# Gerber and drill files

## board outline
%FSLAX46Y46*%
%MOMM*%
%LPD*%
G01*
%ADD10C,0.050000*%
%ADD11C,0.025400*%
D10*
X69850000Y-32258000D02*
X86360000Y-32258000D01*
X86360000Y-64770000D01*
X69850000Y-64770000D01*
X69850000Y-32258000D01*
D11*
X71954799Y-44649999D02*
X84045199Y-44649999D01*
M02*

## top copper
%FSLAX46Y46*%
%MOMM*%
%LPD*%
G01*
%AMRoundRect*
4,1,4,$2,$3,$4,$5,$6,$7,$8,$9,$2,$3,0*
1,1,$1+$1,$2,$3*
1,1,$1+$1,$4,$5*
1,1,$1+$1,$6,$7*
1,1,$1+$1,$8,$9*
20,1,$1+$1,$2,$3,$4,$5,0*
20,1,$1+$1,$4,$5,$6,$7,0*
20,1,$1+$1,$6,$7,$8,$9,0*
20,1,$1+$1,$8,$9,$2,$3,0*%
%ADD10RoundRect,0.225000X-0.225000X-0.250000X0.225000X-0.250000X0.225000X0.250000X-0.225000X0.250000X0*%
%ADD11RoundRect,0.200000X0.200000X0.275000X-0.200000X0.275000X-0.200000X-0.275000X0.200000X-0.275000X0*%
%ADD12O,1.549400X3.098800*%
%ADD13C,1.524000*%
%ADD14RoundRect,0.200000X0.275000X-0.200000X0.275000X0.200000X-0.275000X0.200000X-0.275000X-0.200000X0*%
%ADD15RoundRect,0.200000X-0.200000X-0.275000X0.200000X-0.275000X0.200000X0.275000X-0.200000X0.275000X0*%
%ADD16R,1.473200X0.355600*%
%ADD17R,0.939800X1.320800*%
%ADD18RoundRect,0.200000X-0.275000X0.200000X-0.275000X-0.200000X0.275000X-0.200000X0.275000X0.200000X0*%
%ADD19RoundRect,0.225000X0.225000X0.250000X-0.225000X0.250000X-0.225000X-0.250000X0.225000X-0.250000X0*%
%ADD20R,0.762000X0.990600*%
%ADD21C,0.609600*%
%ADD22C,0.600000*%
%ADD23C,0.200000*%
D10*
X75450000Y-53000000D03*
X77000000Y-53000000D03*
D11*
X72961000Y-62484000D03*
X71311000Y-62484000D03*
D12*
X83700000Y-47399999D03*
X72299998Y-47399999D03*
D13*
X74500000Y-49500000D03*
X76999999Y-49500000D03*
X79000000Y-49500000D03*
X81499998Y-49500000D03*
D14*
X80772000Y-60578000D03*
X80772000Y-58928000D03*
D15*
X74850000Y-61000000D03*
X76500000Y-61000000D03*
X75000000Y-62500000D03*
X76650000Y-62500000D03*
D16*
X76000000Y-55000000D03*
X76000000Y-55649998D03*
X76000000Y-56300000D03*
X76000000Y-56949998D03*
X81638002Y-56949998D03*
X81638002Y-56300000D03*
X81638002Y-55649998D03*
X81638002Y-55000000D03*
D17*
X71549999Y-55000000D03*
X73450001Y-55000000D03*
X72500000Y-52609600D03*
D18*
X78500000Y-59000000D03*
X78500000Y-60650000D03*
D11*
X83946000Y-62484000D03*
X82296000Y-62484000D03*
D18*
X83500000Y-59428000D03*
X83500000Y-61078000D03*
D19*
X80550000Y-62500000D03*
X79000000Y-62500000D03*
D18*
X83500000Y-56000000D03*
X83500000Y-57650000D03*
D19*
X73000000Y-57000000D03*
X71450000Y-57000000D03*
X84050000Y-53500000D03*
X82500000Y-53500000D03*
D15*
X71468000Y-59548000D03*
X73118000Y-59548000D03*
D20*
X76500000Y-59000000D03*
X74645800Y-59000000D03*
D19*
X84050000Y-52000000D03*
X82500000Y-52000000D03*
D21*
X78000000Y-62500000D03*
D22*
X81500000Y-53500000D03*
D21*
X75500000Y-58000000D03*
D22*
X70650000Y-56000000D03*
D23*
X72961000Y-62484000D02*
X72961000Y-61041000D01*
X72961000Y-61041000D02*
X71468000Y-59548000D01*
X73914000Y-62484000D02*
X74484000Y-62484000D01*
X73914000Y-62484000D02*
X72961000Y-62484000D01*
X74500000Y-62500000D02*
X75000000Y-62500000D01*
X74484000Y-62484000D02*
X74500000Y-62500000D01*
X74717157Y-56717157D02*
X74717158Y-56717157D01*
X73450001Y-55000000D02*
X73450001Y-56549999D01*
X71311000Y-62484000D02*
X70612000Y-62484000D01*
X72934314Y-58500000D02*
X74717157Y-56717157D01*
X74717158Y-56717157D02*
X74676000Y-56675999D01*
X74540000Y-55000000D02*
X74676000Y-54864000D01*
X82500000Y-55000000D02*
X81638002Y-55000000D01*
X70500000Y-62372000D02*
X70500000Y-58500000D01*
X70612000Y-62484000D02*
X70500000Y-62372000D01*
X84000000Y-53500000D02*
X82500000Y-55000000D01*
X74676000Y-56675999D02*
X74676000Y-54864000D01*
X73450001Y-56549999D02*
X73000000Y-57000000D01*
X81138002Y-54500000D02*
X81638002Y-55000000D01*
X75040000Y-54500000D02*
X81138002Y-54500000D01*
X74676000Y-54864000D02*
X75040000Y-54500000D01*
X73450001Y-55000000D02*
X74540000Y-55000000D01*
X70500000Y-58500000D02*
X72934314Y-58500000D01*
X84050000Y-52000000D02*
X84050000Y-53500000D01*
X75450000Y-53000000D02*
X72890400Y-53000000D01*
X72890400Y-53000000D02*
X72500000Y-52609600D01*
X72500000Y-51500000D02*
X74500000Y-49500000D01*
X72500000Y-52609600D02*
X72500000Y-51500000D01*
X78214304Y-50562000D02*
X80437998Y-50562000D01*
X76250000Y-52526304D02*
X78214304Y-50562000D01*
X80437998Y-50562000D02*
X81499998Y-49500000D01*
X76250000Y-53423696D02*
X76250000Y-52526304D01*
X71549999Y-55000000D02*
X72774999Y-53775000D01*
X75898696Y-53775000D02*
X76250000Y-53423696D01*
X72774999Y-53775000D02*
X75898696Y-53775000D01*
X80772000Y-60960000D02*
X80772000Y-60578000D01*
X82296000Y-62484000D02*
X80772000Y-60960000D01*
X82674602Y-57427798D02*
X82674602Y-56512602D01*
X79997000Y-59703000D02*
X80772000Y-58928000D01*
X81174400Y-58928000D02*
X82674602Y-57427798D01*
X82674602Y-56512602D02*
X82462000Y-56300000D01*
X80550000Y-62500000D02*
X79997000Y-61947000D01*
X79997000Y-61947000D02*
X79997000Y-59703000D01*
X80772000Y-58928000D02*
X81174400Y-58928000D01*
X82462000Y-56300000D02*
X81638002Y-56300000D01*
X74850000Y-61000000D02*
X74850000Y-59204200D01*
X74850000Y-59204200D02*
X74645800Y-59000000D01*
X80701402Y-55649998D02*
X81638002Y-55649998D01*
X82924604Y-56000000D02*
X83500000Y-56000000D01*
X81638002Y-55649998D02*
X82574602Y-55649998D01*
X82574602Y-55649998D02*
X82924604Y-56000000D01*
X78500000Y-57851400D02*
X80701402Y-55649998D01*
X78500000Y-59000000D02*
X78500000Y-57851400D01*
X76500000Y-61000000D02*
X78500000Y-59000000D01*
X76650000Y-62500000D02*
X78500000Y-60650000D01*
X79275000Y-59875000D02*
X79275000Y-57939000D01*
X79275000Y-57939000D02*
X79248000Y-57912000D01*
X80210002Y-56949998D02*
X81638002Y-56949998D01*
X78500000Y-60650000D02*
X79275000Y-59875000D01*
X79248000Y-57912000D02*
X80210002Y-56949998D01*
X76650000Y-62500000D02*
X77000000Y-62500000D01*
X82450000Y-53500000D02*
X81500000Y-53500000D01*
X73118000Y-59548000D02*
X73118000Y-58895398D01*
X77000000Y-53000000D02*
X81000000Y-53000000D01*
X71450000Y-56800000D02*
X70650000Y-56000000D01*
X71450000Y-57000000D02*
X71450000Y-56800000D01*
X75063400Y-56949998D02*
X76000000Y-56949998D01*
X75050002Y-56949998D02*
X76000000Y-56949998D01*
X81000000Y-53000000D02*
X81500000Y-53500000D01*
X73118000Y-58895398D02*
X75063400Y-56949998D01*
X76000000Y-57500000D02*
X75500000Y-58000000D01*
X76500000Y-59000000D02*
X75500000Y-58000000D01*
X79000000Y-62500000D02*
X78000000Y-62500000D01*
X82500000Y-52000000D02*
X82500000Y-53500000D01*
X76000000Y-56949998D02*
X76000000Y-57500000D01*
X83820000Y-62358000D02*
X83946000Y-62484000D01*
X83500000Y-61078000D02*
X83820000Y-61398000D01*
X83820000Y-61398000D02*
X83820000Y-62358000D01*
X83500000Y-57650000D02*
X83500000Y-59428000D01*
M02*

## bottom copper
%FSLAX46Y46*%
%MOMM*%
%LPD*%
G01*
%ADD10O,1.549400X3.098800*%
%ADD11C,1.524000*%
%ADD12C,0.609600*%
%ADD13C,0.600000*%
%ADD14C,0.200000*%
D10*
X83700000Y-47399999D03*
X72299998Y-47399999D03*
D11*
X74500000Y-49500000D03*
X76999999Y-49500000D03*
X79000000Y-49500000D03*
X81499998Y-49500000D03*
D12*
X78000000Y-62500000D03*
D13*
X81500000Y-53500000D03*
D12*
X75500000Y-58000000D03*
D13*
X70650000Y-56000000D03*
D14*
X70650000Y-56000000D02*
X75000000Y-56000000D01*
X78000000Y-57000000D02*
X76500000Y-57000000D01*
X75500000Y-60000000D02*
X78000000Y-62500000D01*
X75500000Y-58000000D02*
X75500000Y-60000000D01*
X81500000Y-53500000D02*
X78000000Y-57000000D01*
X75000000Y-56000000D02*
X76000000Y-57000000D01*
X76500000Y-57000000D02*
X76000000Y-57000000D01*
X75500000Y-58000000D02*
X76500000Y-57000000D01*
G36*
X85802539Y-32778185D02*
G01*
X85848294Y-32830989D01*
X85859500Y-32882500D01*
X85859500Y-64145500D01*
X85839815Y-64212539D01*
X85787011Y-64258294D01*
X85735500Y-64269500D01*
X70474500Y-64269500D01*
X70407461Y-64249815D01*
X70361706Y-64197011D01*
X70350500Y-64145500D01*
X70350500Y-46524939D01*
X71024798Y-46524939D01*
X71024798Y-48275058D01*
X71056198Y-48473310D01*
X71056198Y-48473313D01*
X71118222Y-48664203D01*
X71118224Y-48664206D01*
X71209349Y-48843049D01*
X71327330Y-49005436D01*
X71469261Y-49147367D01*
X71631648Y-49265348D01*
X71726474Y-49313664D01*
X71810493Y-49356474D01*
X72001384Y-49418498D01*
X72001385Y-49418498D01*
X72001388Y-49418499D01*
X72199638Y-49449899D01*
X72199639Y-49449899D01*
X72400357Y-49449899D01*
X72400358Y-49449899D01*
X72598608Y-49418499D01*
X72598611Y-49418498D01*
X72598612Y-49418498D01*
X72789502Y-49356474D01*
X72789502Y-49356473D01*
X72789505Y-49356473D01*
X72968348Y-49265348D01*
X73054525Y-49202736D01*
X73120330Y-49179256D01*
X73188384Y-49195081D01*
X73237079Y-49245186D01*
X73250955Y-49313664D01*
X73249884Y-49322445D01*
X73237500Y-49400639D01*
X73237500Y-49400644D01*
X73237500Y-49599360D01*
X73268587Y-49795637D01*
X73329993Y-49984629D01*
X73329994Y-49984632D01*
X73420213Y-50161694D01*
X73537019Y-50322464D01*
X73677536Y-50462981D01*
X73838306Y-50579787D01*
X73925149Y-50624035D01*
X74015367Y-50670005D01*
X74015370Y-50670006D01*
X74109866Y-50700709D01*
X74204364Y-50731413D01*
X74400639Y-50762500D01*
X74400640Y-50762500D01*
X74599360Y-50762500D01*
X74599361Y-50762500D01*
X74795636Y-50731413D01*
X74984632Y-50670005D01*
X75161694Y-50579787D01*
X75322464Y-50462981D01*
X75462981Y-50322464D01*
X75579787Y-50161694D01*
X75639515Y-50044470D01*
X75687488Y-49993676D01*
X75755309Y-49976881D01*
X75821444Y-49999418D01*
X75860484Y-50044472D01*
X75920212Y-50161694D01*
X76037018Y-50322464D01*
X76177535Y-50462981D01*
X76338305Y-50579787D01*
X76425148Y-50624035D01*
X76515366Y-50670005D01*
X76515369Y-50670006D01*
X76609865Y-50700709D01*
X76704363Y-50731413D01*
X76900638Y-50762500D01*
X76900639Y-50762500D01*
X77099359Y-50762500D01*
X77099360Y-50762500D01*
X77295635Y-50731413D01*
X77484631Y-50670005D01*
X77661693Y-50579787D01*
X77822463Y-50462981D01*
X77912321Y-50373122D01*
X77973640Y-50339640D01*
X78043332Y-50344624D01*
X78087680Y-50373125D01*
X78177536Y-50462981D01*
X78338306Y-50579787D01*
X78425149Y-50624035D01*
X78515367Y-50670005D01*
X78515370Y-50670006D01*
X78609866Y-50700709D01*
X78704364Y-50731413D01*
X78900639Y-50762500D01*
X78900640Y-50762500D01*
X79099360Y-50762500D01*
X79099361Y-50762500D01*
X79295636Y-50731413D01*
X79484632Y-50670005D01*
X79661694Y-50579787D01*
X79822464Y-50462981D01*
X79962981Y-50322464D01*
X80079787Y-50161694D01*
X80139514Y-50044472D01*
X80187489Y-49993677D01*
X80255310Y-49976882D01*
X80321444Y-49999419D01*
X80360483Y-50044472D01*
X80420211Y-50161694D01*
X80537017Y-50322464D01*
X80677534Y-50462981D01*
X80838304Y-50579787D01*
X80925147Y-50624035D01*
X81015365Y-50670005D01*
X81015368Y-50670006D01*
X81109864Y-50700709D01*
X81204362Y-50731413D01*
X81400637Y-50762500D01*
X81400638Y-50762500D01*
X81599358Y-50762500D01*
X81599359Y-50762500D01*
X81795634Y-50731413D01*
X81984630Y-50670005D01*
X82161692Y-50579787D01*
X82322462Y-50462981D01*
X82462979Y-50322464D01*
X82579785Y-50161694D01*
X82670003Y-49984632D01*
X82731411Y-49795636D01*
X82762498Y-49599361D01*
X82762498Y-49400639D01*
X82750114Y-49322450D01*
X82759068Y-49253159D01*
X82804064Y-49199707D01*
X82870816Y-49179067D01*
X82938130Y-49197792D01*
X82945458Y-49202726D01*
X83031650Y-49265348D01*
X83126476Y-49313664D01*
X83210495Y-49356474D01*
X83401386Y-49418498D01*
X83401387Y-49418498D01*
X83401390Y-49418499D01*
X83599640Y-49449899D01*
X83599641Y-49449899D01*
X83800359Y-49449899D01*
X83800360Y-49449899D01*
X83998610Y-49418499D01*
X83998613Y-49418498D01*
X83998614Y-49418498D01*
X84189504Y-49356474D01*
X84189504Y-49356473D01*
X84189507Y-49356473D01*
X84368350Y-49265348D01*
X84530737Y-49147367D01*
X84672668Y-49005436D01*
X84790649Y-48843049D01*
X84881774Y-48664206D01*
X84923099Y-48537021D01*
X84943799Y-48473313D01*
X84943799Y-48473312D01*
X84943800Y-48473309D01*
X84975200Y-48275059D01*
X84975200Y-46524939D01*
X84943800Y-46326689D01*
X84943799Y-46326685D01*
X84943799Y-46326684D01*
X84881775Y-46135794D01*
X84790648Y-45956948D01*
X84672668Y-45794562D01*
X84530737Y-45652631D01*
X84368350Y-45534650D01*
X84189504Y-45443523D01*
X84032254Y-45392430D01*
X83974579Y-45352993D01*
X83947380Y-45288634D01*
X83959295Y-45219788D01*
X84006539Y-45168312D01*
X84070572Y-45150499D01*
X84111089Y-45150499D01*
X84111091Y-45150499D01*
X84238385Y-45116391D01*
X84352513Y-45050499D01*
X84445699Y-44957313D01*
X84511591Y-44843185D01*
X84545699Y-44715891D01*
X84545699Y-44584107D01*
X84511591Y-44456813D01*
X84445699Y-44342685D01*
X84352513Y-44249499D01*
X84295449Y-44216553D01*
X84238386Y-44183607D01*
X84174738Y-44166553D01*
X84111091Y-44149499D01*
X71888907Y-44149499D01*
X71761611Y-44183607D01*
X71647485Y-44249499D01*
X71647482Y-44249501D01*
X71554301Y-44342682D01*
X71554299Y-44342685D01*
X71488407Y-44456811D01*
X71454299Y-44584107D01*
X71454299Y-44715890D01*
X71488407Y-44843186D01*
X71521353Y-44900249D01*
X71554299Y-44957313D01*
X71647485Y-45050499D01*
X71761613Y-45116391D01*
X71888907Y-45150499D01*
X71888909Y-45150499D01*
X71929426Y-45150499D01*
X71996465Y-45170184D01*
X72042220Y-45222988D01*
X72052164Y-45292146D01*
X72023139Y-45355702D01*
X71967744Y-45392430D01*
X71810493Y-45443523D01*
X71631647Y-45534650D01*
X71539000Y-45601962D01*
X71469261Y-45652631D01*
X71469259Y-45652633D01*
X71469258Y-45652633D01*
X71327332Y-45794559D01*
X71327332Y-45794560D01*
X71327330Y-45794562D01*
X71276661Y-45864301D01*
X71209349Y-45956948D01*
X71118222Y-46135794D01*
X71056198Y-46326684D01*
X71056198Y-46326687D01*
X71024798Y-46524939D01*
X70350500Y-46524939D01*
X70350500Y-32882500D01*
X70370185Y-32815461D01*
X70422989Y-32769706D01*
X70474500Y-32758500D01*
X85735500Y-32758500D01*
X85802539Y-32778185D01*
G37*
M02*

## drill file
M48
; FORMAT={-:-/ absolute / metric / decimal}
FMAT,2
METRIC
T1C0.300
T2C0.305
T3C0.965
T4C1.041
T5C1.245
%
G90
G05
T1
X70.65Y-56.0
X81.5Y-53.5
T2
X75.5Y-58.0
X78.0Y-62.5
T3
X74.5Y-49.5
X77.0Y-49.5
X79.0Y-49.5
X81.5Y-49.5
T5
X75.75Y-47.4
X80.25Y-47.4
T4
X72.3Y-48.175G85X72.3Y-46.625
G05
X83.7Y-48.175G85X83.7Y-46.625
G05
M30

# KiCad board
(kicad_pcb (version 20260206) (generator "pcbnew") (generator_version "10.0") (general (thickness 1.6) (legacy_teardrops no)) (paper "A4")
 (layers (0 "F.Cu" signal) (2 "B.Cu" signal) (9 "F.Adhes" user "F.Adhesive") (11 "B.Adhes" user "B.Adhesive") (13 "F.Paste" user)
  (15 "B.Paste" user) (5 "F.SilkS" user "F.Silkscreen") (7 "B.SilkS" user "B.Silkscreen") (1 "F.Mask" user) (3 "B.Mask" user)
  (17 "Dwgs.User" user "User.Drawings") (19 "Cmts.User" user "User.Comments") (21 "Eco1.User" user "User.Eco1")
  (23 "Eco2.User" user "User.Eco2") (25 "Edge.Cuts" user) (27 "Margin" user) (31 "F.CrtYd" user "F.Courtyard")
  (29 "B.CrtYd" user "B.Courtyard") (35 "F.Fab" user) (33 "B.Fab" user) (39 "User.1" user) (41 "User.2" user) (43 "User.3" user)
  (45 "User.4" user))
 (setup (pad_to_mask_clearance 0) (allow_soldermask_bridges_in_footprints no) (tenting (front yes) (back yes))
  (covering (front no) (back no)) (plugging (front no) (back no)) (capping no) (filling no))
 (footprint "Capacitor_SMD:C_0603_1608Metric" (layer "F.Cu") (at 76.225 53)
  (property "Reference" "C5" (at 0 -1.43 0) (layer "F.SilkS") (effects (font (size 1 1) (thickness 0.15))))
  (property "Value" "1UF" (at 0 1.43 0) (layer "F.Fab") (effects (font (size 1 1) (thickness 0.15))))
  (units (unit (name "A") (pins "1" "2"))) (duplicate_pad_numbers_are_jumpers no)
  (pad "1" smd roundrect (at -0.775 0) (size 0.9 0.95) (layers "F.Cu" "F.Mask" "F.Paste") (roundrect_rratio 0.25) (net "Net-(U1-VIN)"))
  (pad "2" smd roundrect (at 0.775 0) (size 0.9 0.95) (layers "F.Cu" "F.Mask" "F.Paste") (roundrect_rratio 0.25) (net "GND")))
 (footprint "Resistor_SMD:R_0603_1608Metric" (layer "F.Cu") (at 72.136 62.484 180)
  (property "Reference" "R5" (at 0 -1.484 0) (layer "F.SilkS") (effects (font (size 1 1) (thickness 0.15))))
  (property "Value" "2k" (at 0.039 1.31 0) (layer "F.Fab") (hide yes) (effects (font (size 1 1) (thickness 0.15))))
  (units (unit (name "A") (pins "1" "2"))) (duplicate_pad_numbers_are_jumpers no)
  (pad "1" smd roundrect (at -0.825 0 180) (size 0.8 0.95) (layers "F.Cu" "F.Mask" "F.Paste") (roundrect_rratio 0.25) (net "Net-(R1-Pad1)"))
  (pad "2" smd roundrect (at 0.825 0 180) (size 0.8 0.95) (layers "F.Cu" "F.Mask" "F.Paste") (roundrect_rratio 0.25) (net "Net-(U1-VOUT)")))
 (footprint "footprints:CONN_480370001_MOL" (layer "F.Cu") (at 74.5 49.5 180)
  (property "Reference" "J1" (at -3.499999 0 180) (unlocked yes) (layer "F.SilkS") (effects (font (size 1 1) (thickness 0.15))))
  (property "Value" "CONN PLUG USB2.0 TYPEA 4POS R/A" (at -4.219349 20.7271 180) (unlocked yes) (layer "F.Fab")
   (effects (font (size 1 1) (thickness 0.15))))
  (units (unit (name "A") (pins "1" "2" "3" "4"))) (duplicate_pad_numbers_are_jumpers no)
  (fp_line (start 2.545201 4.850001) (end -9.545199 4.850001) (stroke (width 0.0254) (type solid)) (layer "Edge.Cuts"))
  (pad "" np_thru_hole oval (at -9.2 2.100001 180) (size 1.5494 3.0988) (drill oval 1.0414 2.5908) (layers "*.Cu" "*.Mask"))
  (pad "" np_thru_hole circle (at -5.75 2.100001 180) (size 1.2446 1.2446) (drill 1.2446) (layers))
  (pad "" np_thru_hole circle (at -1.249999 2.100001 180) (size 1.2446 1.2446) (drill 1.2446) (layers))
  (pad "" np_thru_hole oval (at 2.200002 2.100001 180) (size 1.5494 3.0988) (drill oval 1.0414 2.5908) (layers "*.Cu" "*.Mask"))
  (pad "1" thru_hole circle (at 0 0 180) (size 1.524 1.524) (drill 0.9652) (layers "*.Cu" "*.Mask") (remove_unused_layers no)
   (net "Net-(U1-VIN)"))
  (pad "2" thru_hole circle (at -2.499999 0 180) (size 1.524 1.524) (drill 0.9652) (layers "*.Cu" "*.Mask") (remove_unused_layers no)
   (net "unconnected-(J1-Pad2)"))
  (pad "3" thru_hole circle (at -4.5 0 180) (size 1.524 1.524) (drill 0.9652) (layers "*.Cu" "*.Mask") (remove_unused_layers no)
   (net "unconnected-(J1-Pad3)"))
  (pad "4" thru_hole circle (at -6.999998 0 180) (size 1.524 1.524) (drill 0.9652) (layers "*.Cu" "*.Mask") (remove_unused_layers no)
   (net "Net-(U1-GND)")))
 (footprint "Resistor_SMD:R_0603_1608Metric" (layer "F.Cu") (at 80.772 59.753 90)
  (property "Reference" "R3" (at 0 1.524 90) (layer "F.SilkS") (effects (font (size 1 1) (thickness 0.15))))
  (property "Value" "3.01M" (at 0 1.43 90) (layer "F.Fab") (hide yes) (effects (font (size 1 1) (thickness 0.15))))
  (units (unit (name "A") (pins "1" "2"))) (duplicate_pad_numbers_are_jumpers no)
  (pad "1" smd roundrect (at -0.825 0 90) (size 0.8 0.95) (layers "F.Cu" "F.Mask" "F.Paste") (roundrect_rratio 0.25) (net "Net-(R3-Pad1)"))
  (pad "2" smd roundrect (at 0.825 0 90) (size 0.8 0.95) (layers "F.Cu" "F.Mask" "F.Paste") (roundrect_rratio 0.25) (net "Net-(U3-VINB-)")))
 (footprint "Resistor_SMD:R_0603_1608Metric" (layer "F.Cu") (at 75.675 61)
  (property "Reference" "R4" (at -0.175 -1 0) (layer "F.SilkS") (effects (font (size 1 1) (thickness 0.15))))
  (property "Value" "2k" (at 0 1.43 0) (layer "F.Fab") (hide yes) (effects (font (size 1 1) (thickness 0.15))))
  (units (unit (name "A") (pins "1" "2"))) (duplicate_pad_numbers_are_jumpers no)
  (pad "1" smd roundrect (at -0.825 0) (size 0.8 0.95) (layers "F.Cu" "F.Mask" "F.Paste") (roundrect_rratio 0.25) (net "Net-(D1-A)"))
  (pad "2" smd roundrect (at 0.825 0) (size 0.8 0.95) (layers "F.Cu" "F.Mask" "F.Paste") (roundrect_rratio 0.25) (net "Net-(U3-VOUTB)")))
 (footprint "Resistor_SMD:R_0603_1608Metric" (layer "F.Cu") (at 75.825 62.5)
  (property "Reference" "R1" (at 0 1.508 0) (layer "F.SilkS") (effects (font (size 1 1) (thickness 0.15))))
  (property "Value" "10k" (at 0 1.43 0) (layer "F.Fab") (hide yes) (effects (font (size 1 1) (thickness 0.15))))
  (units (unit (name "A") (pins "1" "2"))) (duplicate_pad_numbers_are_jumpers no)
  (pad "1" smd roundrect (at -0.825 0) (size 0.8 0.95) (layers "F.Cu" "F.Mask" "F.Paste") (roundrect_rratio 0.25) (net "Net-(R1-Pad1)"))
  (pad "2" smd roundrect (at 0.825 0) (size 0.8 0.95) (layers "F.Cu" "F.Mask" "F.Paste") (roundrect_rratio 0.25) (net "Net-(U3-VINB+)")))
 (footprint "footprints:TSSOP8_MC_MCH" (layer "F.Cu") (at 78.819001 55.974999)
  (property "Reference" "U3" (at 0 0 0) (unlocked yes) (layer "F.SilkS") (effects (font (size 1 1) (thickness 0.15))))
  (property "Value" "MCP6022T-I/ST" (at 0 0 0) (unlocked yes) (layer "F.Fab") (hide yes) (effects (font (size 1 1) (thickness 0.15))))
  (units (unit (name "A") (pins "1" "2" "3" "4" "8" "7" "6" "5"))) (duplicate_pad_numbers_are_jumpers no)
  (pad "1" smd rect (at -2.819001 -0.974999) (size 1.4732 0.3556) (layers "F.Cu" "F.Mask" "F.Paste") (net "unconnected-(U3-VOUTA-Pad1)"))
  (pad "2" smd rect (at -2.819001 -0.325001) (size 1.4732 0.3556) (layers "F.Cu" "F.Mask" "F.Paste") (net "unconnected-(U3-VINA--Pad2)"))
  (pad "3" smd rect (at -2.819001 0.325001) (size 1.4732 0.3556) (layers "F.Cu" "F.Mask" "F.Paste") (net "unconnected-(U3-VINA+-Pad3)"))
  (pad "4" smd rect (at -2.819001 0.974999) (size 1.4732 0.3556) (layers "F.Cu" "F.Mask" "F.Paste") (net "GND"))
  (pad "5" smd rect (at 2.819001 0.974999) (size 1.4732 0.3556) (layers "F.Cu" "F.Mask" "F.Paste") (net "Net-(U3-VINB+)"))
  (pad "6" smd rect (at 2.819001 0.325001) (size 1.4732 0.3556) (layers "F.Cu" "F.Mask" "F.Paste") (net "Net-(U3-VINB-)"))
  (pad "7" smd rect (at 2.819001 -0.325001) (size 1.4732 0.3556) (layers "F.Cu" "F.Mask" "F.Paste") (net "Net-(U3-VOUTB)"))
  (pad "8" smd rect (at 2.819001 -0.974999) (size 1.4732 0.3556) (layers "F.Cu" "F.Mask" "F.Paste") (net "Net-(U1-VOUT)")))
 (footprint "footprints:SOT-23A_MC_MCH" (layer "F.Cu") (at 72.5 53.8048)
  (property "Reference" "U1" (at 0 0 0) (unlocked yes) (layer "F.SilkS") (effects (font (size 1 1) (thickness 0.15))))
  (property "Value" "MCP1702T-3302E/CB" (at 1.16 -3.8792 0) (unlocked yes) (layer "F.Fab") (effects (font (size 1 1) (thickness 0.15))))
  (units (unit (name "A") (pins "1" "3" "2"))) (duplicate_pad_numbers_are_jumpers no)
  (pad "1" smd rect (at -0.950001 1.1952) (size 0.9398 1.3208) (layers "F.Cu" "F.Mask" "F.Paste") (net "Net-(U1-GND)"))
  (pad "2" smd rect (at 0.950001 1.1952) (size 0.9398 1.3208) (layers "F.Cu" "F.Mask" "F.Paste") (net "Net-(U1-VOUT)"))
  (pad "3" smd rect (at 0 -1.1952) (size 0.9398 1.3208) (layers "F.Cu" "F.Mask" "F.Paste") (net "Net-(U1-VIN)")))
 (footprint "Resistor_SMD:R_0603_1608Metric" (layer "F.Cu") (at 78.5 59.825 -90)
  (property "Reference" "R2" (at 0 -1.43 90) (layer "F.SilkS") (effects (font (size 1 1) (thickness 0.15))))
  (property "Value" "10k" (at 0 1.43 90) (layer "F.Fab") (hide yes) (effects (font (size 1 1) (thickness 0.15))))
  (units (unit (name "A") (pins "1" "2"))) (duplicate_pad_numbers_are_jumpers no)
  (pad "1" smd roundrect (at -0.825 0 270) (size 0.8 0.95) (layers "F.Cu" "F.Mask" "F.Paste") (roundrect_rratio 0.25) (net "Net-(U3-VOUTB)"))
  (pad "2" smd roundrect (at 0.825 0 270) (size 0.8 0.95) (layers "F.Cu" "F.Mask" "F.Paste") (roundrect_rratio 0.25) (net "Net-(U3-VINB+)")))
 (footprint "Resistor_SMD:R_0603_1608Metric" (layer "F.Cu") (at 83.121 62.484 180)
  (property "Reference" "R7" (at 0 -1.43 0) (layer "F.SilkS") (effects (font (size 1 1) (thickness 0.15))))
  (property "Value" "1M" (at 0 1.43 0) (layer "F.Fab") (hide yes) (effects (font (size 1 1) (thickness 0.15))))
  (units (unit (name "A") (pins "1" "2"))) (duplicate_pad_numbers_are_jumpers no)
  (pad "1" smd roundrect (at -0.825 0 180) (size 0.8 0.95) (layers "F.Cu" "F.Mask" "F.Paste") (roundrect_rratio 0.25) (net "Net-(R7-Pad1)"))
  (pad "2" smd roundrect (at 0.825 0 180) (size 0.8 0.95) (layers "F.Cu" "F.Mask" "F.Paste") (roundrect_rratio 0.25) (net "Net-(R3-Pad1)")))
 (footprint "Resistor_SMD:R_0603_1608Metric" (layer "F.Cu") (at 83.5 60.253 -90)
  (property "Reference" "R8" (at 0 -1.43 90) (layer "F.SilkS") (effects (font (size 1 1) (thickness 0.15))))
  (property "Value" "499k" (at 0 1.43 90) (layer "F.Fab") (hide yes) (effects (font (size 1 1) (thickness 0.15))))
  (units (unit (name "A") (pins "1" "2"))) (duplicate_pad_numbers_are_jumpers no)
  (pad "1" smd roundrect (at -0.825 0 270) (size 0.8 0.95) (layers "F.Cu" "F.Mask" "F.Paste") (roundrect_rratio 0.25) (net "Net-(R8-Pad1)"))
  (pad "2" smd roundrect (at 0.825 0 270) (size 0.8 0.95) (layers "F.Cu" "F.Mask" "F.Paste") (roundrect_rratio 0.25) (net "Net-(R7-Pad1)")))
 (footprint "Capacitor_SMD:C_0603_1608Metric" (layer "F.Cu") (at 79.775 62.5 180)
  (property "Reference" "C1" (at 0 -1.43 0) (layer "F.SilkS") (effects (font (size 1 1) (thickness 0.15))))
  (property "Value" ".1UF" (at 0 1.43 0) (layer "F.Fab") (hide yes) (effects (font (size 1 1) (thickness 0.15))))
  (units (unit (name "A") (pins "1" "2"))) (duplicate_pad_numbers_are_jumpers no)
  (pad "1" smd roundrect (at -0.775 0 180) (size 0.9 0.95) (layers "F.Cu" "F.Mask" "F.Paste") (roundrect_rratio 0.25) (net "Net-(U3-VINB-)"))
  (pad "2" smd roundrect (at 0.775 0 180) (size 0.9 0.95) (layers "F.Cu" "F.Mask" "F.Paste") (roundrect_rratio 0.25) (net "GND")))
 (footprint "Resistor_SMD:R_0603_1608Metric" (layer "F.Cu") (at 83.5 56.825 -90)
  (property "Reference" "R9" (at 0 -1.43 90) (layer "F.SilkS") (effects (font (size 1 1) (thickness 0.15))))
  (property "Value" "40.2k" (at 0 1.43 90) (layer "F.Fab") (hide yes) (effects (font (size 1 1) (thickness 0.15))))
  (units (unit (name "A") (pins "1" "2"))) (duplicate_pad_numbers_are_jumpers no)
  (pad "1" smd roundrect (at -0.825 0 270) (size 0.8 0.95) (layers "F.Cu" "F.Mask" "F.Paste") (roundrect_rratio 0.25) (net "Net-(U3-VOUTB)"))
  (pad "2" smd roundrect (at 0.825 0 270) (size 0.8 0.95) (layers "F.Cu" "F.Mask" "F.Paste") (roundrect_rratio 0.25) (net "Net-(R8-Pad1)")))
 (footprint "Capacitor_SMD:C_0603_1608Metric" (layer "F.Cu") (at 72.225 57 180)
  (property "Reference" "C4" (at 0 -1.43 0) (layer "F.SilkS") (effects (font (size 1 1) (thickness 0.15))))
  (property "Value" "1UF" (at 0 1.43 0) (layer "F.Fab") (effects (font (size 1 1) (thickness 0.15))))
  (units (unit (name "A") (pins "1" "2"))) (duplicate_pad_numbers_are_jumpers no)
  (pad "1" smd roundrect (at -0.775 0 180) (size 0.9 0.95) (layers "F.Cu" "F.Mask" "F.Paste") (roundrect_rratio 0.25) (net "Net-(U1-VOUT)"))
  (pad "2" smd roundrect (at 0.775 0 180) (size 0.9 0.95) (layers "F.Cu" "F.Mask" "F.Paste") (roundrect_rratio 0.25) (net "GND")))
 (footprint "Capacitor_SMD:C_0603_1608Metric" (layer "F.Cu") (at 83.275 53.5 180)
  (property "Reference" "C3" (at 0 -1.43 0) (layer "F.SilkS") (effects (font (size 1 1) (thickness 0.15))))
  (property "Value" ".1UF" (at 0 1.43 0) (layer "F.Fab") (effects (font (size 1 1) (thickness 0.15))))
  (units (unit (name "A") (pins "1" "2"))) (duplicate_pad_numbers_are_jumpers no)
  (pad "1" smd roundrect (at -0.775 0 180) (size 0.9 0.95) (layers "F.Cu" "F.Mask" "F.Paste") (roundrect_rratio 0.25) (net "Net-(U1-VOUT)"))
  (pad "2" smd roundrect (at 0.775 0 180) (size 0.9 0.95) (layers "F.Cu" "F.Mask" "F.Paste") (roundrect_rratio 0.25) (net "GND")))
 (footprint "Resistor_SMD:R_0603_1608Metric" (layer "F.Cu") (at 72.293 59.548)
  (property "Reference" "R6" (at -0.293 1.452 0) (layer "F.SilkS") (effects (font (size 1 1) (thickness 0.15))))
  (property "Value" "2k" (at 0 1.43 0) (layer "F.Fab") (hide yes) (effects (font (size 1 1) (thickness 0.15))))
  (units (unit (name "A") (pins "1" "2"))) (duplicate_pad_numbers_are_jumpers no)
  (pad "1" smd roundrect (at -0.825 0) (size 0.8 0.95) (layers "F.Cu" "F.Mask" "F.Paste") (roundrect_rratio 0.25) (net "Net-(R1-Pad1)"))
  (pad "2" smd roundrect (at 0.825 0) (size 0.8 0.95) (layers "F.Cu" "F.Mask" "F.Paste") (roundrect_rratio 0.25) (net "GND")))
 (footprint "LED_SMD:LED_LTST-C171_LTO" (layer "F.Cu") (at 75.5729 59 180)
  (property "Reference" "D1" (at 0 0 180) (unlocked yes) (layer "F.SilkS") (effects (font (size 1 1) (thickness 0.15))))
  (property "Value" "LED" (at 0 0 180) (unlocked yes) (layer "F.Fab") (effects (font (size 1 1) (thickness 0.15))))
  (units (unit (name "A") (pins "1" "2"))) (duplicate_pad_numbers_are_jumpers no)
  (pad "1" smd rect (at -0.9271 0 180) (size 0.762 0.9906) (layers "F.Cu" "F.Mask" "F.Paste") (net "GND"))
  (pad "2" smd rect (at 0.9271 0 180) (size 0.762 0.9906) (layers "F.Cu" "F.Mask" "F.Paste") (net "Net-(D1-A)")))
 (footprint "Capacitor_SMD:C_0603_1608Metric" (layer "F.Cu") (at 83.275 52 180)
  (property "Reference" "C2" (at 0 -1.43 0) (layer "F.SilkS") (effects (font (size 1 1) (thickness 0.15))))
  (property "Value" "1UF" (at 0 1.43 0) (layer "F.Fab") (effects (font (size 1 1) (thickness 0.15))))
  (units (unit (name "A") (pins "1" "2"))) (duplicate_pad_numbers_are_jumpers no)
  (pad "1" smd roundrect (at -0.775 0 180) (size 0.9 0.95) (layers "F.Cu" "F.Mask" "F.Paste") (roundrect_rratio 0.25) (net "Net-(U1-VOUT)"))
  (pad "2" smd roundrect (at 0.775 0 180) (size 0.9 0.95) (layers "F.Cu" "F.Mask" "F.Paste") (roundrect_rratio 0.25) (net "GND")))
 (gr_rect (start 69.85 32.258) (end 86.36 64.77) (stroke (width 0.05) (type default)) (fill no) (layer "Edge.Cuts"))
 (segment (start 72.961 62.484) (end 72.961 61.041) (width 0.2) (layer "F.Cu") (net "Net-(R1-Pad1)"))
 (segment (start 72.961 61.041) (end 71.468 59.548) (width 0.2) (layer "F.Cu") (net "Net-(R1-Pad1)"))
 (segment (start 73.914 62.484) (end 74.484 62.484) (width 0.2) (layer "F.Cu") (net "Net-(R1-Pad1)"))
 (segment (start 73.914 62.484) (end 72.961 62.484) (width 0.2) (layer "F.Cu") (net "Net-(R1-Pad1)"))
 (segment (start 74.5 62.5) (end 75 62.5) (width 0.2) (layer "F.Cu") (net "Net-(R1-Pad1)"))
 (segment (start 74.484 62.484) (end 74.5 62.5) (width 0.2) (layer "F.Cu") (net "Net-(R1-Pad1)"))
 (segment (start 74.717157 56.717157) (end 74.717158 56.717157) (width 0.2) (layer "F.Cu") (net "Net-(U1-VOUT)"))
 (segment (start 73.450001 55) (end 73.450001 56.549999) (width 0.2) (layer "F.Cu") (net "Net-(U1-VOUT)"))
 (segment (start 71.311 62.484) (end 70.612 62.484) (width 0.2) (layer "F.Cu") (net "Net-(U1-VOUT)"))
 (segment (start 72.934314 58.5) (end 74.717157 56.717157) (width 0.2) (layer "F.Cu") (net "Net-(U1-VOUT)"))
 (segment (start 74.717158 56.717157) (end 74.676 56.675999) (width 0.2) (layer "F.Cu") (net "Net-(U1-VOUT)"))
 (segment (start 74.54 55) (end 74.676 54.864) (width 0.2) (layer "F.Cu") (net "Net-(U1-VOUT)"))
 (segment (start 82.5 55) (end 81.638002 55) (width 0.2) (layer "F.Cu") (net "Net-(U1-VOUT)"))
 (segment (start 70.5 62.372) (end 70.5 58.5) (width 0.2) (layer "F.Cu") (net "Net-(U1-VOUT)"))
 (segment (start 70.612 62.484) (end 70.5 62.372) (width 0.2) (layer "F.Cu") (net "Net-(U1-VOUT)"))
 (segment (start 84 53.5) (end 82.5 55) (width 0.2) (layer "F.Cu") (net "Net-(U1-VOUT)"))
 (segment (start 74.676 56.675999) (end 74.676 54.864) (width 0.2) (layer "F.Cu") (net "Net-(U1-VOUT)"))
 (segment (start 73.450001 56.549999) (end 73 57) (width 0.2) (layer "F.Cu") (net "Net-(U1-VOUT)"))
 (segment (start 81.138002 54.5) (end 81.638002 55) (width 0.2) (layer "F.Cu") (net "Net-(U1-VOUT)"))
 (segment (start 75.04 54.5) (end 81.138002 54.5) (width 0.2) (layer "F.Cu") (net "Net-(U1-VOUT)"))
 (segment (start 74.676 54.864) (end 75.04 54.5) (width 0.2) (layer "F.Cu") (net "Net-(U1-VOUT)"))
 (segment (start 73.450001 55) (end 74.54 55) (width 0.2) (layer "F.Cu") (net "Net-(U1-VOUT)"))
 (segment (start 70.5 58.5) (end 72.934314 58.5) (width 0.2) (layer "F.Cu") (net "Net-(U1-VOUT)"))
 (segment (start 84.05 52) (end 84.05 53.5) (width 0.2) (layer "F.Cu") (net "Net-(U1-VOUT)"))
 (segment (start 75.45 53) (end 72.8904 53) (width 0.2) (layer "F.Cu") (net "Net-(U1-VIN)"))
 (segment (start 72.8904 53) (end 72.5 52.6096) (width 0.2) (layer "F.Cu") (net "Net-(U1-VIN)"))
 (segment (start 72.5 51.5) (end 74.5 49.5) (width 0.2) (layer "F.Cu") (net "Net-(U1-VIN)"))
 (segment (start 72.5 52.6096) (end 72.5 51.5) (width 0.2) (layer "F.Cu") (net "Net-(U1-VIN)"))
 (segment (start 78.214304 50.562) (end 80.437998 50.562) (width 0.2) (layer "F.Cu") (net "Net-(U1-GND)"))
 (segment (start 76.25 52.526304) (end 78.214304 50.562) (width 0.2) (layer "F.Cu") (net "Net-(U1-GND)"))
 (segment (start 80.437998 50.562) (end 81.499998 49.5) (width 0.2) (layer "F.Cu") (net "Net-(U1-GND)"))
 (segment (start 76.25 53.423696) (end 76.25 52.526304) (width 0.2) (layer "F.Cu") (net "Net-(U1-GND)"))
 (segment (start 71.549999 55) (end 72.774999 53.775) (width 0.2) (layer "F.Cu") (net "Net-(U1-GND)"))
 (segment (start 75.898696 53.775) (end 76.25 53.423696) (width 0.2) (layer "F.Cu") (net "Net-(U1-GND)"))
 (segment (start 72.774999 53.775) (end 75.898696 53.775) (width 0.2) (layer "F.Cu") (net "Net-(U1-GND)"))
 (segment (start 80.772 60.96) (end 80.772 60.578) (width 0.2) (layer "F.Cu") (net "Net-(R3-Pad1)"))
 (segment (start 82.296 62.484) (end 80.772 60.96) (width 0.2) (layer "F.Cu") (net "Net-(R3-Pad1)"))
 (segment (start 82.674602 57.427798) (end 82.674602 56.512602) (width 0.2) (layer "F.Cu") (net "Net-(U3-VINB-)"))
 (segment (start 79.997 59.703) (end 80.772 58.928) (width 0.2) (layer "F.Cu") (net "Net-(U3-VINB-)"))
 (segment (start 81.1744 58.928) (end 82.674602 57.427798) (width 0.2) (layer "F.Cu") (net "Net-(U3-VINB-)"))
 (segment (start 82.674602 56.512602) (end 82.462 56.3) (width 0.2) (layer "F.Cu") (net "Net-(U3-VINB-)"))
 (segment (start 80.55 62.5) (end 79.997 61.947) (width 0.2) (layer "F.Cu") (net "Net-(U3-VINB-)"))
 (segment (start 79.997 61.947) (end 79.997 59.703) (width 0.2) (layer "F.Cu") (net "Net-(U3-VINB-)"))
 (segment (start 80.772 58.928) (end 81.1744 58.928) (width 0.2) (layer "F.Cu") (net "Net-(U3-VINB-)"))
 (segment (start 82.462 56.3) (end 81.638002 56.3) (width 0.2) (layer "F.Cu") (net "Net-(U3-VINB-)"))
 (segment (start 74.85 61) (end 74.85 59.2042) (width 0.2) (layer "F.Cu") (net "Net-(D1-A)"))
 (segment (start 74.85 59.2042) (end 74.6458 59) (width 0.2) (layer "F.Cu") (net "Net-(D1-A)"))
 (segment (start 80.701402 55.649998) (end 81.638002 55.649998) (width 0.2) (layer "F.Cu") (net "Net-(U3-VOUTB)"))
 (segment (start 82.924604 56) (end 83.5 56) (width 0.2) (layer "F.Cu") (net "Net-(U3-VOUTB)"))
 (segment (start 81.638002 55.649998) (end 82.574602 55.649998) (width 0.2) (layer "F.Cu") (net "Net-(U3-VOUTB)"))
 (segment (start 82.574602 55.649998) (end 82.924604 56) (width 0.2) (layer "F.Cu") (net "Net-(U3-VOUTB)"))
 (segment (start 78.5 57.8514) (end 80.701402 55.649998) (width 0.2) (layer "F.Cu") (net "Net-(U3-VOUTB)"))
 (segment (start 78.5 59) (end 78.5 57.8514) (width 0.2) (layer "F.Cu") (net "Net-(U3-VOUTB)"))
 (segment (start 76.5 61) (end 78.5 59) (width 0.2) (layer "F.Cu") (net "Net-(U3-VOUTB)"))
 (segment (start 76.65 62.5) (end 78.5 60.65) (width 0.2) (layer "F.Cu") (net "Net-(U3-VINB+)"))
 (segment (start 79.275 59.875) (end 79.275 57.939) (width 0.2) (layer "F.Cu") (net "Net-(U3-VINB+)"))
 (segment (start 79.275 57.939) (end 79.248 57.912) (width 0.2) (layer "F.Cu") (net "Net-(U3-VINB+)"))
 (segment (start 80.210002 56.949998) (end 81.638002 56.949998) (width 0.2) (layer "F.Cu") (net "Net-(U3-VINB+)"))
 (segment (start 78.5 60.65) (end 79.275 59.875) (width 0.2) (layer "F.Cu") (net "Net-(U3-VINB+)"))
 (segment (start 79.248 57.912) (end 80.210002 56.949998) (width 0.2) (layer "F.Cu") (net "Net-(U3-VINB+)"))
 (segment (start 76.65 62.5) (end 77 62.5) (width 0.2) (layer "F.Cu") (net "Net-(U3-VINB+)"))
 (segment (start 82.45 53.5) (end 81.5 53.5) (width 0.2) (layer "F.Cu") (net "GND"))
 (segment (start 73.118 59.548) (end 73.118 58.895398) (width 0.2) (layer "F.Cu") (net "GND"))
 (segment (start 77 53) (end 81 53) (width 0.2) (layer "F.Cu") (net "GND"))
 (segment (start 71.45 56.8) (end 70.65 56) (width 0.2) (layer "F.Cu") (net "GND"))
 (segment (start 71.45 57) (end 71.45 56.8) (width 0.2) (layer "F.Cu") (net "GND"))
 (segment (start 75.0634 56.949998) (end 76 56.949998) (width 0.2) (layer "F.Cu") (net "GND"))
 (segment (start 75.050002 56.949998) (end 76 56.949998) (width 0.2) (layer "F.Cu") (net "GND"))
 (segment (start 81 53) (end 81.5 53.5) (width 0.2) (layer "F.Cu") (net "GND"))
 (segment (start 73.118 58.895398) (end 75.0634 56.949998) (width 0.2) (layer "F.Cu") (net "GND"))
 (segment (start 76 57.5) (end 75.5 58) (width 0.2) (layer "F.Cu") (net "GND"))
 (segment (start 76.5 59) (end 75.5 58) (width 0.2) (layer "F.Cu") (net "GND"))
 (segment (start 79 62.5) (end 78 62.5) (width 0.2) (layer "F.Cu") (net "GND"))
 (segment (start 82.5 52) (end 82.5 53.5) (width 0.2) (layer "F.Cu") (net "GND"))
 (segment (start 76 56.949998) (end 76 57.5) (width 0.2) (layer "F.Cu") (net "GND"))
 (via (at 78 62.5) (size 0.6096) (drill 0.3048) (layers "F.Cu" "B.Cu") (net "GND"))
 (via (at 81.5 53.5) (size 0.6) (drill 0.3) (layers "F.Cu" "B.Cu") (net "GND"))
 (via (at 75.5 58) (size 0.6096) (drill 0.3048) (layers "F.Cu" "B.Cu") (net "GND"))
 (via (at 70.65 56) (size 0.6) (drill 0.3) (layers "F.Cu" "B.Cu") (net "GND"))
 (segment (start 70.65 56) (end 75 56) (width 0.2) (layer "B.Cu") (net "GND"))
 (segment (start 78 57) (end 76.5 57) (width 0.2) (layer "B.Cu") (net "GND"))
 (segment (start 75.5 60) (end 78 62.5) (width 0.2) (layer "B.Cu") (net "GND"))
 (segment (start 75.5 58) (end 75.5 60) (width 0.2) (layer "B.Cu") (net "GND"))
 (segment (start 81.5 53.5) (end 78 57) (width 0.2) (layer "B.Cu") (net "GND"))
 (segment (start 75 56) (end 76 57) (width 0.2) (layer "B.Cu") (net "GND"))
 (segment (start 76.5 57) (end 76 57) (width 0.2) (layer "B.Cu") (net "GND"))
 (segment (start 75.5 58) (end 76.5 57) (width 0.2) (layer "B.Cu") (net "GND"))
 (segment (start 83.82 62.358) (end 83.946 62.484) (width 0.2) (layer "F.Cu") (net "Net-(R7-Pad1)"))
 (segment (start 83.5 61.078) (end 83.82 61.398) (width 0.2) (layer "F.Cu") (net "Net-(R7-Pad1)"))
 (segment (start 83.82 61.398) (end 83.82 62.358) (width 0.2) (layer "F.Cu") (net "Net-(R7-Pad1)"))
 (segment (start 83.5 57.65) (end 83.5 59.428) (width 0.2) (layer "F.Cu") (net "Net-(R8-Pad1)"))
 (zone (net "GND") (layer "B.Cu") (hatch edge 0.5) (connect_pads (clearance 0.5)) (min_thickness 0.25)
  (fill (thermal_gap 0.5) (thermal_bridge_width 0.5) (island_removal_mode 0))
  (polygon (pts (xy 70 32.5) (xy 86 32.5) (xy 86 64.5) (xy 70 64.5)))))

